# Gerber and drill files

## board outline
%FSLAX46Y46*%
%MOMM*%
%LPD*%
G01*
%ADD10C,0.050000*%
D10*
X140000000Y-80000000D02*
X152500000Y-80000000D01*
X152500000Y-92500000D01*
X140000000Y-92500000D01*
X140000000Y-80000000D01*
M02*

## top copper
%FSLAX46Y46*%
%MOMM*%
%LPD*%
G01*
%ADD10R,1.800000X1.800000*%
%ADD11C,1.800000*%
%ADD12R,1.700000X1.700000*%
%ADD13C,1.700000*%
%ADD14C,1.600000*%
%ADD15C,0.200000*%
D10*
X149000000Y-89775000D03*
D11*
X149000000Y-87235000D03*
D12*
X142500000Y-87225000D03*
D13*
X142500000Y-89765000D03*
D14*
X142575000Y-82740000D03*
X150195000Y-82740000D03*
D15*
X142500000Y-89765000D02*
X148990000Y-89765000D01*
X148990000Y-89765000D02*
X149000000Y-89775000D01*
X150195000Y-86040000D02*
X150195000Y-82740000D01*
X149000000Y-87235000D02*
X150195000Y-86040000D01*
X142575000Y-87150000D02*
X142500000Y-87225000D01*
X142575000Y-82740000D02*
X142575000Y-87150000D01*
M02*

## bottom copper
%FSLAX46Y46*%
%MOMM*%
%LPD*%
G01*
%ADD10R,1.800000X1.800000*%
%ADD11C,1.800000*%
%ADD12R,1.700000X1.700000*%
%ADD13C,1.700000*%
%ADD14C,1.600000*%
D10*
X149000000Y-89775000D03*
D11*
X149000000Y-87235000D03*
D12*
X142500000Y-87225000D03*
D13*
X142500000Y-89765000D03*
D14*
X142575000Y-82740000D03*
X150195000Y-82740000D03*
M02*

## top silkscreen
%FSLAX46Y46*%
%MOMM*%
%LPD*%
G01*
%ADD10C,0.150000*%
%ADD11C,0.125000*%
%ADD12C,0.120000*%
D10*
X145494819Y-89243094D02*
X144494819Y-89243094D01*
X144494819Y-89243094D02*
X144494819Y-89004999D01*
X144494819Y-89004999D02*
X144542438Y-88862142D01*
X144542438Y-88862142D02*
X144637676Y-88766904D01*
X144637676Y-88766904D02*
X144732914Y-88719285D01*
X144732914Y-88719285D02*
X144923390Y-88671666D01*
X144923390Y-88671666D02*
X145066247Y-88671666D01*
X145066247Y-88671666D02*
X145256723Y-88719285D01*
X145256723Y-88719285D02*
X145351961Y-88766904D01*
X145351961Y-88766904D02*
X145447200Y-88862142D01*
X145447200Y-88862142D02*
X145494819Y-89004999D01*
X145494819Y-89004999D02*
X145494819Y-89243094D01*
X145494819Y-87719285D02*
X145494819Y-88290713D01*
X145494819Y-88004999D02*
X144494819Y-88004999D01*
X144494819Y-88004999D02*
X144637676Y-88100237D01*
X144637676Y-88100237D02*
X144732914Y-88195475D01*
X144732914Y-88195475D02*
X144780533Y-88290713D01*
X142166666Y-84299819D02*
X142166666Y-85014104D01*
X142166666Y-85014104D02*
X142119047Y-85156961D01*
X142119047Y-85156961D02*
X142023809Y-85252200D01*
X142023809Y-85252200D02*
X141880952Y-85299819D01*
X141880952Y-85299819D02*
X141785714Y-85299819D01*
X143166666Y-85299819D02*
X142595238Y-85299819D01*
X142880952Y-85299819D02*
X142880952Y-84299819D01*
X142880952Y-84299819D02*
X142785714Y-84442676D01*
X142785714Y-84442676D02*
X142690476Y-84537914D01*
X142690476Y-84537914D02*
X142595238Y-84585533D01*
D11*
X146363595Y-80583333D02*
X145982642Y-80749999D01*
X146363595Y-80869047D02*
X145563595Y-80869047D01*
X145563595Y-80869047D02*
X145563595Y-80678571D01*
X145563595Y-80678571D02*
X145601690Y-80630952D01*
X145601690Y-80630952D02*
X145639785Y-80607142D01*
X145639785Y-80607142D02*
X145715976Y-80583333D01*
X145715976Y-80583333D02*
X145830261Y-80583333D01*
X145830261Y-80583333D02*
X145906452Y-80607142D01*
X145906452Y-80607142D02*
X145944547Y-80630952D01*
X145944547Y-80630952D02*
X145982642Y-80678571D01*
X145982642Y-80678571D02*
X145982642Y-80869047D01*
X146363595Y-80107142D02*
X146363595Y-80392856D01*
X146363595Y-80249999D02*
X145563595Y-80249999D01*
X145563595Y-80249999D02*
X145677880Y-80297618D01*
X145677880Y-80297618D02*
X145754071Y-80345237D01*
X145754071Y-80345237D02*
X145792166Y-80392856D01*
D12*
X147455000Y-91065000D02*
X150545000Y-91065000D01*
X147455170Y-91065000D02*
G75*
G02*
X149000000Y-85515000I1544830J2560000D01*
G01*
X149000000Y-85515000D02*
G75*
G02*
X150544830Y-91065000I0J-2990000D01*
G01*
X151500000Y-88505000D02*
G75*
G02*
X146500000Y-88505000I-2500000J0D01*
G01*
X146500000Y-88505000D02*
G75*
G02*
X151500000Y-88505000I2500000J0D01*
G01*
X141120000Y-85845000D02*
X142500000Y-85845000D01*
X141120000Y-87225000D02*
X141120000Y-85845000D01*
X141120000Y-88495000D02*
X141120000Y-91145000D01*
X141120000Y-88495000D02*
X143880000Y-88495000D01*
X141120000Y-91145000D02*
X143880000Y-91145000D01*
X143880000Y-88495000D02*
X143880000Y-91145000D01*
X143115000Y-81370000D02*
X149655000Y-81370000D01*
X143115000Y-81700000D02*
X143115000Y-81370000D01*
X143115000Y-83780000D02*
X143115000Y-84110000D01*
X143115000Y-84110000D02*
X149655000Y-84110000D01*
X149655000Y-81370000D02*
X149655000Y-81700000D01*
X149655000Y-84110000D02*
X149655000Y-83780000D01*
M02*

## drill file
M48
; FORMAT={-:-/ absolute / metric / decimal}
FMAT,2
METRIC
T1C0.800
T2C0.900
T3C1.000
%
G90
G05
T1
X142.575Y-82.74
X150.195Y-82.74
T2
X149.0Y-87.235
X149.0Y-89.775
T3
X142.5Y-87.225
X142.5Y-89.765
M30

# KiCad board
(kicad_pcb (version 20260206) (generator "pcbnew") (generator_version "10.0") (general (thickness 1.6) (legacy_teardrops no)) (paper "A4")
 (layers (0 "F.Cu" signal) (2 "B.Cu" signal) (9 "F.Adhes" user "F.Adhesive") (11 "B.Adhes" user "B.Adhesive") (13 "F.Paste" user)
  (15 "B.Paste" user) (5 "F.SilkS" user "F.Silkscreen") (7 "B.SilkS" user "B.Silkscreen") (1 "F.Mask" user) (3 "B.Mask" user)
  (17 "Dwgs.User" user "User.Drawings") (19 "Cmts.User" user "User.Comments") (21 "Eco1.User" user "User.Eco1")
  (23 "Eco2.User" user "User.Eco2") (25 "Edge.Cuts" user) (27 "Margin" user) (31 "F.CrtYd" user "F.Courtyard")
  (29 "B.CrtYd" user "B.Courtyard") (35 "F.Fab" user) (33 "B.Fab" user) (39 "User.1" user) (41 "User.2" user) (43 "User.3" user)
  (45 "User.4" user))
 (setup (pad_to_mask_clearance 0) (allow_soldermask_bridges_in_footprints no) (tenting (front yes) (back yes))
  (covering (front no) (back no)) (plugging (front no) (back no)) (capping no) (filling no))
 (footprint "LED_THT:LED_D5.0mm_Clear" (layer "F.Cu") (at 149 89.775 90)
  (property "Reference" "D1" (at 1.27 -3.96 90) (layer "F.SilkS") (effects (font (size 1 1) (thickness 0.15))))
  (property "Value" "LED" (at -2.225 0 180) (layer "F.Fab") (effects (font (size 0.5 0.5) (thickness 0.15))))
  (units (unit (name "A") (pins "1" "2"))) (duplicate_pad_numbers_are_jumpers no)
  (fp_line (start -1.29 -1.545) (end -1.29 1.545) (stroke (width 0.12) (type solid)) (layer "F.SilkS"))
  (fp_arc (start -1.29 -1.54483) (mid 2.071779 -2.880495) (end 4.26 0) (stroke (width 0.12) (type solid)) (layer "F.SilkS"))
  (fp_arc (start 4.26 0) (mid 2.071779 2.880495) (end -1.29 1.54483) (stroke (width 0.12) (type solid)) (layer "F.SilkS"))
  (fp_circle (center 1.27 0) (end 3.77 0) (stroke (width 0.12) (type solid)) (fill no) (layer "F.SilkS"))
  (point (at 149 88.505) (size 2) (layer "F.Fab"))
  (pad "1" thru_hole rect (at 0 0 90) (size 1.8 1.8) (drill 0.9) (layers "*.Cu" "*.Mask") (remove_unused_layers no) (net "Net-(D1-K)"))
  (pad "2" thru_hole circle (at 2.54 0 90) (size 1.8 1.8) (drill 0.9) (layers "*.Cu" "*.Mask") (remove_unused_layers no) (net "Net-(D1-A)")))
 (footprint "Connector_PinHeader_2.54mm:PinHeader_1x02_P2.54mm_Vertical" (layer "F.Cu") (at 142.5 87.225)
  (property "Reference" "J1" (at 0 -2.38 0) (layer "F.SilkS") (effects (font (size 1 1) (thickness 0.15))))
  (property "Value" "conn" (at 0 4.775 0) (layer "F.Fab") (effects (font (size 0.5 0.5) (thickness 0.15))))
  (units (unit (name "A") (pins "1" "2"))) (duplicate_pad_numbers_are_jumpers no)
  (fp_line (start -1.38 -1.38) (end 0 -1.38) (stroke (width 0.12) (type solid)) (layer "F.SilkS"))
  (fp_line (start -1.38 0) (end -1.38 -1.38) (stroke (width 0.12) (type solid)) (layer "F.SilkS"))
  (fp_line (start -1.38 1.27) (end -1.38 3.92) (stroke (width 0.12) (type solid)) (layer "F.SilkS"))
  (fp_line (start -1.38 1.27) (end 1.38 1.27) (stroke (width 0.12) (type solid)) (layer "F.SilkS"))
  (fp_line (start -1.38 3.92) (end 1.38 3.92) (stroke (width 0.12) (type solid)) (layer "F.SilkS"))
  (fp_line (start 1.38 1.27) (end 1.38 3.92) (stroke (width 0.12) (type solid)) (layer "F.SilkS"))
  (pad "1" thru_hole rect (at 0 0) (size 1.7 1.7) (drill 1) (layers "*.Cu" "*.Mask") (remove_unused_layers no) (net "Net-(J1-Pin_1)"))
  (pad "2" thru_hole circle (at 0 2.54) (size 1.7 1.7) (drill 1) (layers "*.Cu" "*.Mask") (remove_unused_layers no) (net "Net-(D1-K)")))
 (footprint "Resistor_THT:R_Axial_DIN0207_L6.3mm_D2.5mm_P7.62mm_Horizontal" (layer "F.Cu") (at 142.575 82.74)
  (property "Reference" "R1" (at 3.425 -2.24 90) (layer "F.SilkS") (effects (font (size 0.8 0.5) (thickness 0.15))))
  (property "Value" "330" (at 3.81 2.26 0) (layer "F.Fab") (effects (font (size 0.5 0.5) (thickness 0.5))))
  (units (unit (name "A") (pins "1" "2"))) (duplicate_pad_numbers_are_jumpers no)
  (fp_line (start 0.54 -1.37) (end 7.08 -1.37) (stroke (width 0.12) (type solid)) (layer "F.SilkS"))
  (fp_line (start 0.54 -1.04) (end 0.54 -1.37) (stroke (width 0.12) (type solid)) (layer "F.SilkS"))
  (fp_line (start 0.54 1.04) (end 0.54 1.37) (stroke (width 0.12) (type solid)) (layer "F.SilkS"))
  (fp_line (start 0.54 1.37) (end 7.08 1.37) (stroke (width 0.12) (type solid)) (layer "F.SilkS"))
  (fp_line (start 7.08 -1.37) (end 7.08 -1.04) (stroke (width 0.12) (type solid)) (layer "F.SilkS"))
  (fp_line (start 7.08 1.37) (end 7.08 1.04) (stroke (width 0.12) (type solid)) (layer "F.SilkS"))
  (pad "1" thru_hole circle (at 0 0) (size 1.6 1.6) (drill 0.8) (layers "*.Cu" "*.Mask") (remove_unused_layers no) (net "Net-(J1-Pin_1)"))
  (pad "2" thru_hole circle (at 7.62 0) (size 1.6 1.6) (drill 0.8) (layers "*.Cu" "*.Mask") (remove_unused_layers no) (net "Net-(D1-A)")))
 (gr_rect (start 140 80) (end 152.5 92.5) (stroke (width 0.05) (type default)) (fill no) (layer "Edge.Cuts"))
 (segment (start 142.5 89.765) (end 148.99 89.765) (width 0.2) (layer "F.Cu") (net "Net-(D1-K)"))
 (segment (start 148.99 89.765) (end 149 89.775) (width 0.2) (layer "F.Cu") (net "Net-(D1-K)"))
 (segment (start 150.195 86.04) (end 150.195 82.74) (width 0.2) (layer "F.Cu") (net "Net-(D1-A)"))
 (segment (start 149 87.235) (end 150.195 86.04) (width 0.2) (layer "F.Cu") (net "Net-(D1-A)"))
 (segment (start 142.575 87.15) (end 142.5 87.225) (width 0.2) (layer "F.Cu") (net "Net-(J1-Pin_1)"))
 (segment (start 142.575 82.74) (end 142.575 87.15) (width 0.2) (layer "F.Cu") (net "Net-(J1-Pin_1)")))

